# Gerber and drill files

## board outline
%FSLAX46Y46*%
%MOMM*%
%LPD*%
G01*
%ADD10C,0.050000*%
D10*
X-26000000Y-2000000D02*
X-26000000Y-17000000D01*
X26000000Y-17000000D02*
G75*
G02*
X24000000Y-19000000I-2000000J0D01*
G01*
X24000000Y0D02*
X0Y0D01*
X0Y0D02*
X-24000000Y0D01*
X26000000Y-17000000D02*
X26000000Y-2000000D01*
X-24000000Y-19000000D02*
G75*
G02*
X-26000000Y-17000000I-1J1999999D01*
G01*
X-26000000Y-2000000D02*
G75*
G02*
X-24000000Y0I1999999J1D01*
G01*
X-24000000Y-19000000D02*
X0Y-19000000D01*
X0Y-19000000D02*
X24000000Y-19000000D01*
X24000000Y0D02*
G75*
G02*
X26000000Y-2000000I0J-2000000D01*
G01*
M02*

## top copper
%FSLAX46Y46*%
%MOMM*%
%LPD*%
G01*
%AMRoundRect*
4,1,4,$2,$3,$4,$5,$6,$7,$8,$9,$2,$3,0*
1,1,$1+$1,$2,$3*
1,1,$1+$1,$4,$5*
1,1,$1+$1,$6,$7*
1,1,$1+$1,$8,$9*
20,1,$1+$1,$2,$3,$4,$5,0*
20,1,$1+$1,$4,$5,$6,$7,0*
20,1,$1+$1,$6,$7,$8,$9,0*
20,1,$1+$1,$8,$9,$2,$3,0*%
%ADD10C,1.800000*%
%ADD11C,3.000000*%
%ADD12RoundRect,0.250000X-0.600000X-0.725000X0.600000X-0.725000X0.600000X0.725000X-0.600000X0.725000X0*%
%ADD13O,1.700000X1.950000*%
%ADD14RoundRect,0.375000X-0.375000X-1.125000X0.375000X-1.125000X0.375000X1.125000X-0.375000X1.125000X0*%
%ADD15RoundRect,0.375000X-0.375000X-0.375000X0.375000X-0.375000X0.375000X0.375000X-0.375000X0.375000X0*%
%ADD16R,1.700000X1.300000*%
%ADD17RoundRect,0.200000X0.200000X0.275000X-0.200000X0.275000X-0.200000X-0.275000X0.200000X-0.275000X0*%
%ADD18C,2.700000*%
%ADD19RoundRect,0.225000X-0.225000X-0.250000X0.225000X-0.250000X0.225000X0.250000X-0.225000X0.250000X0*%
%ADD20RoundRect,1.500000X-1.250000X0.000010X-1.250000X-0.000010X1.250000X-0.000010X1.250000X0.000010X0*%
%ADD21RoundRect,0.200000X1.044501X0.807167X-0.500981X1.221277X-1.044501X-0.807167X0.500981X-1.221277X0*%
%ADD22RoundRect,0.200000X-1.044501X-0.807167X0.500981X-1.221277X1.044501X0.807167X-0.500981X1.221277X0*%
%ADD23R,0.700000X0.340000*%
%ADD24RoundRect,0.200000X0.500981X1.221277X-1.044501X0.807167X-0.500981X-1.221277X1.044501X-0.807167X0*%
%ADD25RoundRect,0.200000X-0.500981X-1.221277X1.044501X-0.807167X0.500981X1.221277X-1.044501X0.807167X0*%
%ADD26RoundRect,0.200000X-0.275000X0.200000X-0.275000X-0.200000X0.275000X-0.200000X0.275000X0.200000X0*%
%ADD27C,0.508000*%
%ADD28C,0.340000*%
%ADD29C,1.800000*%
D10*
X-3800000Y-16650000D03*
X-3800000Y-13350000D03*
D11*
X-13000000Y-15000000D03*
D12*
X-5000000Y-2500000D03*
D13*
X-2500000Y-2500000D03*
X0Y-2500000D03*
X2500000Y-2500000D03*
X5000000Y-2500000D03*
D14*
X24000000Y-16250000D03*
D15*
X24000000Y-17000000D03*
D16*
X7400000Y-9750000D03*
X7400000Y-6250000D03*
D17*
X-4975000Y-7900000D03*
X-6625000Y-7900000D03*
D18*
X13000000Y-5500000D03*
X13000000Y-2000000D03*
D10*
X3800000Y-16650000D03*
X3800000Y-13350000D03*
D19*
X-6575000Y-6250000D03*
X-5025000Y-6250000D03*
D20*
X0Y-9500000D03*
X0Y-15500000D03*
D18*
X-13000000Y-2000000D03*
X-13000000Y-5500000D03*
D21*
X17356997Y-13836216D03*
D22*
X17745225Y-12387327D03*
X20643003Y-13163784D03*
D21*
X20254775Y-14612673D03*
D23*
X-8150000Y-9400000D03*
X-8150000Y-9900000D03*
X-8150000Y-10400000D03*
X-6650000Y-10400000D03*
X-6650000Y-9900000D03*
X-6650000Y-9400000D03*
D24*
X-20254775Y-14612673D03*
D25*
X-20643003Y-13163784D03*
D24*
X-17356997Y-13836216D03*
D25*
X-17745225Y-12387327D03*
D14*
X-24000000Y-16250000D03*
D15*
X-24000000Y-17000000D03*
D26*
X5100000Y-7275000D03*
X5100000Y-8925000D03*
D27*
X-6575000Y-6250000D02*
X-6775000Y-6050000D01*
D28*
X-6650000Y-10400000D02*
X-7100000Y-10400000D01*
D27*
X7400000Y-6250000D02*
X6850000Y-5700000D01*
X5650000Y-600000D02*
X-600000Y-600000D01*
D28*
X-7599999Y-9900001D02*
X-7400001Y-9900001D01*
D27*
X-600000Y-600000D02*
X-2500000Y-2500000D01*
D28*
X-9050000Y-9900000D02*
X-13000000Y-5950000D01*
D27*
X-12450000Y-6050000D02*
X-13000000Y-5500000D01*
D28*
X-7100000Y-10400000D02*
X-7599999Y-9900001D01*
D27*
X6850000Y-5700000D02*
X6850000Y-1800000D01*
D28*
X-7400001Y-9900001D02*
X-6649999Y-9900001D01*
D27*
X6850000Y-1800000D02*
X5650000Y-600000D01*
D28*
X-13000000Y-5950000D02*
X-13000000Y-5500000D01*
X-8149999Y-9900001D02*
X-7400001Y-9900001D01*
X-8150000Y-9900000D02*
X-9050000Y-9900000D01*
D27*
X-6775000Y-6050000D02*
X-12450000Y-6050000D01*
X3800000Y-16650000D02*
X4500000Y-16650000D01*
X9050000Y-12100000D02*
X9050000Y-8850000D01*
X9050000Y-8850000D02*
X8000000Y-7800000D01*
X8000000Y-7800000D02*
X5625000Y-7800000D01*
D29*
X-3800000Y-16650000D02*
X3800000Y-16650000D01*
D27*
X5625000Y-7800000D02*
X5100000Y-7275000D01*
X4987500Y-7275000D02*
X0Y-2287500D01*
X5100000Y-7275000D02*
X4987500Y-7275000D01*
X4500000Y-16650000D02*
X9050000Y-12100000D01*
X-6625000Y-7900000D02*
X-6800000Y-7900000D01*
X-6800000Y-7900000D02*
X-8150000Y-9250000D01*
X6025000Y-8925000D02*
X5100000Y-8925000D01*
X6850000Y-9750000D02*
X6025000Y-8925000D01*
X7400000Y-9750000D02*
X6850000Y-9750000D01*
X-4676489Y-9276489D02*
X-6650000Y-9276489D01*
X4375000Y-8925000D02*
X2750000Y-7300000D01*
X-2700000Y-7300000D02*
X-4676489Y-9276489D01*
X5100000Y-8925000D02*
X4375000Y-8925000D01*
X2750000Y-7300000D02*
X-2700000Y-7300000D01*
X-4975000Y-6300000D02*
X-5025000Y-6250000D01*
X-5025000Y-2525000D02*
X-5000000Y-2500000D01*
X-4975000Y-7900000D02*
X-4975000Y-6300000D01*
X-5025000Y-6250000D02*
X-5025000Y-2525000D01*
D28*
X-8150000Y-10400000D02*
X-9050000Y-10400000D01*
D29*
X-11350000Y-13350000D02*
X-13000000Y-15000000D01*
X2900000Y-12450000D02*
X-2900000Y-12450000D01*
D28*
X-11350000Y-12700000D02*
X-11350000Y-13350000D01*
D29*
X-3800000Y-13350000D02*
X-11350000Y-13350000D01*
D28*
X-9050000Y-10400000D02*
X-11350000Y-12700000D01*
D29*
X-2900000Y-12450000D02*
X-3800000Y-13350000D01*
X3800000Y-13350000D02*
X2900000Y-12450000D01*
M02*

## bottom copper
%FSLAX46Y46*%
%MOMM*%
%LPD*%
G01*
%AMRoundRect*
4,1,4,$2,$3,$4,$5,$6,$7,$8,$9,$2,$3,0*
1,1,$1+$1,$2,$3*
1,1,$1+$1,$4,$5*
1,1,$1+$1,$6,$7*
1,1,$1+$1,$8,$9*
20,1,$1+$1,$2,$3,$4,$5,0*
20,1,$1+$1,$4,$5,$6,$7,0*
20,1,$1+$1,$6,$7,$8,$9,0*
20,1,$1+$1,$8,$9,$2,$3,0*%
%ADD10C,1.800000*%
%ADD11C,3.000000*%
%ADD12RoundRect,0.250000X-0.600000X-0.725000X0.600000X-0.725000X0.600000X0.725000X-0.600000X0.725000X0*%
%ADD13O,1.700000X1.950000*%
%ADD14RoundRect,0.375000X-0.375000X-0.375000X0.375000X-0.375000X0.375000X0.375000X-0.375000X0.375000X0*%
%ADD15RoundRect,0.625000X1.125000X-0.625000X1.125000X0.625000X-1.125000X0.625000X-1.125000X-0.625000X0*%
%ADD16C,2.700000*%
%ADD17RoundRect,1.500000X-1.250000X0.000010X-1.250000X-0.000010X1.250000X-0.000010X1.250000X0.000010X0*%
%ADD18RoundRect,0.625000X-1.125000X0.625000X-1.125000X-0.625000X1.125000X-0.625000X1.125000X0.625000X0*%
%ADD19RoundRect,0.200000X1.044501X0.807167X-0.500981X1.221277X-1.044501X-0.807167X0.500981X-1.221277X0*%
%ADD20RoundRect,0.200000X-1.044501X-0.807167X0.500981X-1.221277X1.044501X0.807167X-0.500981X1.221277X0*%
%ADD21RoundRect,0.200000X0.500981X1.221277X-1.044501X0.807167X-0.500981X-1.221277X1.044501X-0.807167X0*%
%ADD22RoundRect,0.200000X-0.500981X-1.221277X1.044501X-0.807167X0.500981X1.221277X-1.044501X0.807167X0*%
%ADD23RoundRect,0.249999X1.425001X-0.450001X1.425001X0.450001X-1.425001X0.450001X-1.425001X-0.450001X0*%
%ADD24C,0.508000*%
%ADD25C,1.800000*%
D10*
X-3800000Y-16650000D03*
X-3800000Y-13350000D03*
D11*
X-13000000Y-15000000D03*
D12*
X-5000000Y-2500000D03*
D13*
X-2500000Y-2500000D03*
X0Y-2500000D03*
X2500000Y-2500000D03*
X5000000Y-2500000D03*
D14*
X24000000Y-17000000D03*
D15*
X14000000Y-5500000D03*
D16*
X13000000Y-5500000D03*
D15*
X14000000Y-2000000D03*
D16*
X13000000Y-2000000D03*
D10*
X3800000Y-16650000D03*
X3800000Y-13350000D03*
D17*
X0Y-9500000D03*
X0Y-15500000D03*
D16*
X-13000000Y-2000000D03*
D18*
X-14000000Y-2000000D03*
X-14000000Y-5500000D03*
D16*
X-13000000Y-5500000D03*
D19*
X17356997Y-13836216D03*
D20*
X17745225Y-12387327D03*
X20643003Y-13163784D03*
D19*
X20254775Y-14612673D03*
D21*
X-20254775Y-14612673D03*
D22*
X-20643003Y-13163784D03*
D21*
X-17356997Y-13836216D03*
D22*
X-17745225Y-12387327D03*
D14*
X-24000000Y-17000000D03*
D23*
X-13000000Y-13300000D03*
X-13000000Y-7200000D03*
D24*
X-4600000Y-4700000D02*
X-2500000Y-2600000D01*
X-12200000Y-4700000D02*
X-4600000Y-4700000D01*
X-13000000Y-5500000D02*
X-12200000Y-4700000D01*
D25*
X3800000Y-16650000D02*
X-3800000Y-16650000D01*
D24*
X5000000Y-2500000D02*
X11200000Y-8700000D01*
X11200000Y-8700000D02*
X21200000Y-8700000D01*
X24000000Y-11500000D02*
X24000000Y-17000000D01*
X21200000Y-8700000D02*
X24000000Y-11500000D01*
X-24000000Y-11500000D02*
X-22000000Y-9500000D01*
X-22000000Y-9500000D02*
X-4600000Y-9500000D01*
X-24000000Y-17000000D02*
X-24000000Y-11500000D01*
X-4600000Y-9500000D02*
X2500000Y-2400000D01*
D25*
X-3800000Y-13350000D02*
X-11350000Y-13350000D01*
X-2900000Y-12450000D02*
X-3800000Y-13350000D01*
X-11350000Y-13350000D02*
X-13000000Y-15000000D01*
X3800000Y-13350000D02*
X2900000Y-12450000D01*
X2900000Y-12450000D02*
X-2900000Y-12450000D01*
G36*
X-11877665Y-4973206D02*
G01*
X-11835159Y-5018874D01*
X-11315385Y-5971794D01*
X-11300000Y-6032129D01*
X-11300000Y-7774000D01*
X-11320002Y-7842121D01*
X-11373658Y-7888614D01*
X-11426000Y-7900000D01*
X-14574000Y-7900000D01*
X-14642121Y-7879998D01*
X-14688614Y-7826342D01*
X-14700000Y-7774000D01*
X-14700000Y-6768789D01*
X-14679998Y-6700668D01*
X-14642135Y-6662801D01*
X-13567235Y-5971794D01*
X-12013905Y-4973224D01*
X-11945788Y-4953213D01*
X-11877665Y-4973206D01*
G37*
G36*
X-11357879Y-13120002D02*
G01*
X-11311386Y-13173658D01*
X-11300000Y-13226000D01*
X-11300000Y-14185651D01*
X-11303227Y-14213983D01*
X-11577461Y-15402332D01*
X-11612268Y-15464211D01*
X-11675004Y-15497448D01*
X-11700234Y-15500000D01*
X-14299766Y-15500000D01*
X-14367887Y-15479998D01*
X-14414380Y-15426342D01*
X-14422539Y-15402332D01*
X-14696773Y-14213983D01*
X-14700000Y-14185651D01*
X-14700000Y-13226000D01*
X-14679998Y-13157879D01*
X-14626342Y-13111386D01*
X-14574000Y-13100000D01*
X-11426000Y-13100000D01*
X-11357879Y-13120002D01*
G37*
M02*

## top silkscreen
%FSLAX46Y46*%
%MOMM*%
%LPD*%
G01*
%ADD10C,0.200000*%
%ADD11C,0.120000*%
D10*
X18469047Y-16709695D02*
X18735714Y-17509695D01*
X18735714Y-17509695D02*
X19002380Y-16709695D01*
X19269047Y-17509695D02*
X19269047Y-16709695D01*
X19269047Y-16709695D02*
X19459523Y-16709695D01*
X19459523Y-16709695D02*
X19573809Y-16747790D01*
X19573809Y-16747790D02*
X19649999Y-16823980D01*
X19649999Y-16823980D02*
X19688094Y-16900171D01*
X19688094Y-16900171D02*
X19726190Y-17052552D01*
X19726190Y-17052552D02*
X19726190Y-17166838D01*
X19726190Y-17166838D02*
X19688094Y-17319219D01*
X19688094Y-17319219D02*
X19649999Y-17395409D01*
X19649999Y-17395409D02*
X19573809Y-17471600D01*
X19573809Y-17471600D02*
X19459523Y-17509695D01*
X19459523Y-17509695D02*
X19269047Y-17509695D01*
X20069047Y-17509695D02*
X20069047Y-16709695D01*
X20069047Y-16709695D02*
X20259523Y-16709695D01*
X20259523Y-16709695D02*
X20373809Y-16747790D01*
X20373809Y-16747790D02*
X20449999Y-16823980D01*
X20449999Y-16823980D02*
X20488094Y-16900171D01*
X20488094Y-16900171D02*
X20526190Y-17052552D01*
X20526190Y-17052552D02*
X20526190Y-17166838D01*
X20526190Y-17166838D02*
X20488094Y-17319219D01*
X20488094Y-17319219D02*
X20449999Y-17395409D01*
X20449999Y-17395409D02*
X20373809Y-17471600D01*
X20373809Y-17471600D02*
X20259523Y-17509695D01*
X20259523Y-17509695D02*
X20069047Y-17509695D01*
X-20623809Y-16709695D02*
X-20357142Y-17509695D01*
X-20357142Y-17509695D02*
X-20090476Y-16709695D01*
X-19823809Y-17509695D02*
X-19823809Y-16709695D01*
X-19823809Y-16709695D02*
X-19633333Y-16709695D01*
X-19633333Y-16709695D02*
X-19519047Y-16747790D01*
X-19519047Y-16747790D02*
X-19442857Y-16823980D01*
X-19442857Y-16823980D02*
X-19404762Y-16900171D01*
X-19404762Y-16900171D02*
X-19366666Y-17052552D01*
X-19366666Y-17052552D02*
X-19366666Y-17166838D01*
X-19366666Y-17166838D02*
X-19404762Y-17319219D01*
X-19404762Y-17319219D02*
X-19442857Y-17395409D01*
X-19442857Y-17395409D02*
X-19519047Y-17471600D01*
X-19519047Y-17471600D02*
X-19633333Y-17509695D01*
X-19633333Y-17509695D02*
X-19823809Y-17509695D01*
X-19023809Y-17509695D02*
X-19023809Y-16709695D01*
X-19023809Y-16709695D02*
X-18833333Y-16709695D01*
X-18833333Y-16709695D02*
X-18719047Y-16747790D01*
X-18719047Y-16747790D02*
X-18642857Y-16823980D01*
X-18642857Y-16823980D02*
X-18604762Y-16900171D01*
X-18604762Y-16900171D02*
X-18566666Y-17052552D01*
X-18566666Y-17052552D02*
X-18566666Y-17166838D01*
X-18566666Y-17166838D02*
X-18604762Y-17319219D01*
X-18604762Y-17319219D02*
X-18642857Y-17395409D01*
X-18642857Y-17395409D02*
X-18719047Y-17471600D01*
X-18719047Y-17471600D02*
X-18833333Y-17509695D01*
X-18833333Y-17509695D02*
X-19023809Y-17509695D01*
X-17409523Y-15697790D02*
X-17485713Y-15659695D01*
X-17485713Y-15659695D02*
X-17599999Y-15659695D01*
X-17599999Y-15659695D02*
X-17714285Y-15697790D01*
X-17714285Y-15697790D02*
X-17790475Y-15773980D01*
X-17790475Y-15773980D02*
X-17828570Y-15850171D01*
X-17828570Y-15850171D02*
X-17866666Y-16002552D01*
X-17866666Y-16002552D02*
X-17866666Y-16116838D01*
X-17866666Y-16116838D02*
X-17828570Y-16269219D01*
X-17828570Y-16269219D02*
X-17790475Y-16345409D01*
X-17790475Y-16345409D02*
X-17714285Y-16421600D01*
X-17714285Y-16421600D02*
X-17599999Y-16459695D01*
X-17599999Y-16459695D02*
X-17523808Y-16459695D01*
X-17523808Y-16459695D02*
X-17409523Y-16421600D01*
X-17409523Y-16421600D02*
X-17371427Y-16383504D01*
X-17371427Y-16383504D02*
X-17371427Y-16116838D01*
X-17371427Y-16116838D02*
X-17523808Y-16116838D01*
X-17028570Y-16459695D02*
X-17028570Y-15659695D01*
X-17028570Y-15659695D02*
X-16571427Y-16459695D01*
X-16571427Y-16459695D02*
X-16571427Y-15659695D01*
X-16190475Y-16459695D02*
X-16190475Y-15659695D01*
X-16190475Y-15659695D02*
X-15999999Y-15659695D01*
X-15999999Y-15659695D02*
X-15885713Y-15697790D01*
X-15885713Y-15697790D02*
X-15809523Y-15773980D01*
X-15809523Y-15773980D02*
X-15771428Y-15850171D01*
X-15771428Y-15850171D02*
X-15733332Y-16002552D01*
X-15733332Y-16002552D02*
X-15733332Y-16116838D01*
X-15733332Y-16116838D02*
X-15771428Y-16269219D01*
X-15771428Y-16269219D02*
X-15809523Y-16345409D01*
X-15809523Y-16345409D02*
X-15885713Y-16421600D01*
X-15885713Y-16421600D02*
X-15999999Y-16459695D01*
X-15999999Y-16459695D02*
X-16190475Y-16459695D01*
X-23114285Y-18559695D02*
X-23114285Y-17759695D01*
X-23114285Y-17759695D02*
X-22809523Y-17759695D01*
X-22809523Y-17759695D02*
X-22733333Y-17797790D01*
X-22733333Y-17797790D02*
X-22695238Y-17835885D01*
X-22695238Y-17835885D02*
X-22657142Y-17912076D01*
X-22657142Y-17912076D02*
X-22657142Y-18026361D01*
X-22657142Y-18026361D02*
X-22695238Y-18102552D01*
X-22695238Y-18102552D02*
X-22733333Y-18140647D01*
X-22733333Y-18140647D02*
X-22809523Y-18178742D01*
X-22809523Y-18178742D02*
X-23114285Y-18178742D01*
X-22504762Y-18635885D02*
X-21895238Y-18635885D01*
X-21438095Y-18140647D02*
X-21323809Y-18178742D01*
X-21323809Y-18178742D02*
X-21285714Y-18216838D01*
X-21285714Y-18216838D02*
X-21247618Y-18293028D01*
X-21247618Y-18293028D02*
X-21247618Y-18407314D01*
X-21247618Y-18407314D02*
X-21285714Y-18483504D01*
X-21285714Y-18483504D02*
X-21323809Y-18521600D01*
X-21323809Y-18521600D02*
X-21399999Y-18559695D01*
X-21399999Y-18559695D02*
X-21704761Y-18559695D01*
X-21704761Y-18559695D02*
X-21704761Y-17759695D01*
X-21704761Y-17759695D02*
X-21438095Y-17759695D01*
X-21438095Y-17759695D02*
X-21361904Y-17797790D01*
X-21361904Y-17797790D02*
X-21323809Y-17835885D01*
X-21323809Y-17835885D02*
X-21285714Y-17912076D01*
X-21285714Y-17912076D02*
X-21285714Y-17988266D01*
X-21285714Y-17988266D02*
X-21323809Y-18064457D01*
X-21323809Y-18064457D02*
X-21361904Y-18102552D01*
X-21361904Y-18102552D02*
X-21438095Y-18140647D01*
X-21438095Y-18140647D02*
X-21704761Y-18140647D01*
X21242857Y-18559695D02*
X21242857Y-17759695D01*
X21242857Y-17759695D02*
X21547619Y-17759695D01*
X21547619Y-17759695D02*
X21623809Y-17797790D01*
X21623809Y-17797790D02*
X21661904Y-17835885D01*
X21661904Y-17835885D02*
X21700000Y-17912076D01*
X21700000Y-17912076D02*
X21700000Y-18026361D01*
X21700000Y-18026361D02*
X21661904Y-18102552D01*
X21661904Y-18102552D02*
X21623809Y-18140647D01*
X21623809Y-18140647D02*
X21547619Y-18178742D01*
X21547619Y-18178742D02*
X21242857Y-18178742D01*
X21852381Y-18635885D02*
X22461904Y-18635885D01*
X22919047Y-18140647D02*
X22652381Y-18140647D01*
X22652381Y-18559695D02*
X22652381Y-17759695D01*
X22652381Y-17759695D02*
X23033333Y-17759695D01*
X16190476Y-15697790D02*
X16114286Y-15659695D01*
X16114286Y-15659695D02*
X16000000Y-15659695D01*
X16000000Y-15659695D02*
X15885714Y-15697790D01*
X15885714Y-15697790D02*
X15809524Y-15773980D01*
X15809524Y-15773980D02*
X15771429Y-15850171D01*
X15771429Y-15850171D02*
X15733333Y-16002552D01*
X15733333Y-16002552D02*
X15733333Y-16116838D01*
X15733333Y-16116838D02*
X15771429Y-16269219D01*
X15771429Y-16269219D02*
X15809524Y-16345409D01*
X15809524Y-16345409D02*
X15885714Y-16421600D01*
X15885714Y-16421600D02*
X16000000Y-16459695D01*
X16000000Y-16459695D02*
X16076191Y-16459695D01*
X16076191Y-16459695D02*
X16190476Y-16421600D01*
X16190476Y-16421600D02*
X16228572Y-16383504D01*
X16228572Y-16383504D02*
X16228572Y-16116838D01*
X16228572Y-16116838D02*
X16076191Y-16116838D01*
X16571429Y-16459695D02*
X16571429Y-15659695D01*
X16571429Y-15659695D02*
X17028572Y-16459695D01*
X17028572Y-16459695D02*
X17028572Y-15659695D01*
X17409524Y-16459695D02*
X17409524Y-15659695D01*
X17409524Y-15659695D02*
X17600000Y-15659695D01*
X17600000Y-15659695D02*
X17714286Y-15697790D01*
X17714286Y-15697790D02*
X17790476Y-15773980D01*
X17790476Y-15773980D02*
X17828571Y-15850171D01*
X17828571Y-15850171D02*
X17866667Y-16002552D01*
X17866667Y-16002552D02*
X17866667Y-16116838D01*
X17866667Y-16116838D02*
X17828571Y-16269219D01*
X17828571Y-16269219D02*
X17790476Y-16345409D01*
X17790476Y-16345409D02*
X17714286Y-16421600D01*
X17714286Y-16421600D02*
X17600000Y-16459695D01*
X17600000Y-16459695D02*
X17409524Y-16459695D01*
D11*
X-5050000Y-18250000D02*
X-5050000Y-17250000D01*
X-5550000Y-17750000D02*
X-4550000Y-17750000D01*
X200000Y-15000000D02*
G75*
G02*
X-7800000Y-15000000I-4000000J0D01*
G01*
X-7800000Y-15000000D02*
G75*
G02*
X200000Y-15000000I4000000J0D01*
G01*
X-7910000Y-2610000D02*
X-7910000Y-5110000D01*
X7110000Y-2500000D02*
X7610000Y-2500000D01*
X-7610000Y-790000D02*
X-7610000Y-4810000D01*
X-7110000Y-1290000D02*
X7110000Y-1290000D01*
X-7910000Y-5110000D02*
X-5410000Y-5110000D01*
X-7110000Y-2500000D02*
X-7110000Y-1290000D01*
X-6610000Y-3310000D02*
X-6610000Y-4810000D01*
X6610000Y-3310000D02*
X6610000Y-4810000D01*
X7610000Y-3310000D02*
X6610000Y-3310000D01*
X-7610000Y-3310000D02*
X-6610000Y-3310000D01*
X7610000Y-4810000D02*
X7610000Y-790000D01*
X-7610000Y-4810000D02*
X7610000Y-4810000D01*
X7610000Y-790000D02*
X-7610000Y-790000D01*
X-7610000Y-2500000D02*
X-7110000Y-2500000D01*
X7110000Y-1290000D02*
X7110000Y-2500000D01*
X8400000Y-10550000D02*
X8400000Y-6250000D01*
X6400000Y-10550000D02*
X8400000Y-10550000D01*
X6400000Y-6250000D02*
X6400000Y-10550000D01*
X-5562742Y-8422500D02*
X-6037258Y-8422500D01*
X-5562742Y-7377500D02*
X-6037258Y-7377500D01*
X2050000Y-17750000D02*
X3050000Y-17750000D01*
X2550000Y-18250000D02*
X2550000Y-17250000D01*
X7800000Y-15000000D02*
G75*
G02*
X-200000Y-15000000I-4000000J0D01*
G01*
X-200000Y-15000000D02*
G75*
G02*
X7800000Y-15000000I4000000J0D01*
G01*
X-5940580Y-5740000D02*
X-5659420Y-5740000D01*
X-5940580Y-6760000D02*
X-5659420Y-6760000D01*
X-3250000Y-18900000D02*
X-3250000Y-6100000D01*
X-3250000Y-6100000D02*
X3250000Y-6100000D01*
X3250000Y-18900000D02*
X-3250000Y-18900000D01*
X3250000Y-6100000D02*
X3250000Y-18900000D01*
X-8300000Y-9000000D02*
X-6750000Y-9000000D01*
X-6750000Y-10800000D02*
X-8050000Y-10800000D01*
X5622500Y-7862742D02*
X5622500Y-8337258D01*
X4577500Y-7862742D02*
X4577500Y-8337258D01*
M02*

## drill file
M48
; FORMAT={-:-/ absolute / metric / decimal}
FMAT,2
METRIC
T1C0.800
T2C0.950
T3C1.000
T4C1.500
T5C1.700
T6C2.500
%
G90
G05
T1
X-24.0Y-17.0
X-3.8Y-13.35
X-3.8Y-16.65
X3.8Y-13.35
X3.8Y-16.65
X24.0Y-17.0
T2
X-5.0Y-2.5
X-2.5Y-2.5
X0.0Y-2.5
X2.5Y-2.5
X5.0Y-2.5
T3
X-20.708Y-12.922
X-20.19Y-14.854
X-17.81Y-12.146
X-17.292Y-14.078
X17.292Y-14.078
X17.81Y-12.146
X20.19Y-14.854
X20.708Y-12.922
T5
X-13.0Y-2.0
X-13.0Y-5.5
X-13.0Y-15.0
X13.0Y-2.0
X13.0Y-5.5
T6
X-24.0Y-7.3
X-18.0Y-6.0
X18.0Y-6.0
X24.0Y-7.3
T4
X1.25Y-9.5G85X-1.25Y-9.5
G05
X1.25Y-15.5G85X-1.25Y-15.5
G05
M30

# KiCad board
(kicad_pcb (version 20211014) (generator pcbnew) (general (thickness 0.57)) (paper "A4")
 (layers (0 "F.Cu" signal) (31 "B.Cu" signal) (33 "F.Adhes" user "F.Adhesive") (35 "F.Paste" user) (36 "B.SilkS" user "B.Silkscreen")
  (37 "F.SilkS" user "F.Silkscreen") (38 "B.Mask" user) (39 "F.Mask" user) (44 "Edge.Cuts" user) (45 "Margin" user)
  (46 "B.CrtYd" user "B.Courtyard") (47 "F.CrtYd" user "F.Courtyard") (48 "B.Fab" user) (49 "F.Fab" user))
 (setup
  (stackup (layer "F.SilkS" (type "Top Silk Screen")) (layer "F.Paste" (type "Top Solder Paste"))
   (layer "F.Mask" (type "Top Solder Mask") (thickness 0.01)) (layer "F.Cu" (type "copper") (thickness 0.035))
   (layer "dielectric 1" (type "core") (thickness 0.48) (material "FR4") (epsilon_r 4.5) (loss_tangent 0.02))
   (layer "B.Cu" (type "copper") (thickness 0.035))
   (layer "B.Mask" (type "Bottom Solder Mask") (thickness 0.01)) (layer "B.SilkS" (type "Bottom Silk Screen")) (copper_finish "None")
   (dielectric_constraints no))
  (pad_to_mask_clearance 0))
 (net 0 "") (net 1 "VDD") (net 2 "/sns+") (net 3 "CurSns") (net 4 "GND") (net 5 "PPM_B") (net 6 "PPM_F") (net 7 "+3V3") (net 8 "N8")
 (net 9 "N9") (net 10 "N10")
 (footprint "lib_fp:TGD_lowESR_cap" (layer "F.Cu") (at -3.8 15 90)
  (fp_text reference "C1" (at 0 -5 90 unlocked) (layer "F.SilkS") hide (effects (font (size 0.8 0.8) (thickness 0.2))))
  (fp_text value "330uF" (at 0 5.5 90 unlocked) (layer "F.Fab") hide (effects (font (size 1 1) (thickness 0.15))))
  (fp_line (start -3.25 -1.25) (end -2.25 -1.25) (layer "F.SilkS") (width 0.12))
  (fp_line (start -2.75 -1.75) (end -2.75 -0.75) (layer "F.SilkS") (width 0.12))
  (fp_circle (center 0 0) (end 4 0) (layer "F.SilkS") (width 0.12) (fill none))
  (pad "1" thru_hole circle (at -1.65 0 90) (size 1.8 1.8) (drill 0.8) (layers *.Cu *.Mask) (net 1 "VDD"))
  (pad "2" thru_hole circle (at 1.65 0 90) (size 1.8 1.8) (drill 0.8) (layers *.Cu *.Mask) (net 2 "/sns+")))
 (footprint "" (layer "F.Cu") (at -13 15)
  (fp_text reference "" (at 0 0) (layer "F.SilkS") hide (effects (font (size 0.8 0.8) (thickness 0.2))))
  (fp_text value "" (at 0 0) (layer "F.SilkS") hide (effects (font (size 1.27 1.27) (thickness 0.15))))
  (pad "2" thru_hole circle (at 0 0 270) (size 3 3) (drill 1.7) (layers *.Cu *.Mask) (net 2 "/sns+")))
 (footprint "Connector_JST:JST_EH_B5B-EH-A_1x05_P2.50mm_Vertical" (layer "F.Cu") (at -5 2.5)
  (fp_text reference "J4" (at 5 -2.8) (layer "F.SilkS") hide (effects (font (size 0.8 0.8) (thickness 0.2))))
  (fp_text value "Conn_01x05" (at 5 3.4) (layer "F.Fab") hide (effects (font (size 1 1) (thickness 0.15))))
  (fp_line (start -2.91 0.11) (end -2.91 2.61) (layer "F.SilkS") (width 0.12))
  (fp_line (start 12.11 0) (end 12.61 0) (layer "F.SilkS") (width 0.12))
  (fp_line (start -2.61 -1.71) (end -2.61 2.31) (layer "F.SilkS") (width 0.12))
  (fp_line (start -2.11 -1.21) (end 12.11 -1.21) (layer "F.SilkS") (width 0.12))
  (fp_line (start -2.91 2.61) (end -0.41 2.61) (layer "F.SilkS") (width 0.12))
  (fp_line (start -2.11 0) (end -2.11 -1.21) (layer "F.SilkS") (width 0.12))
  (fp_line (start -1.61 0.81) (end -1.61 2.31) (layer "F.SilkS") (width 0.12))
  (fp_line (start 11.61 0.81) (end 11.61 2.31) (layer "F.SilkS") (width 0.12))
  (fp_line (start 12.61 0.81) (end 11.61 0.81) (layer "F.SilkS") (width 0.12))
  (fp_line (start -2.61 0.81) (end -1.61 0.81) (layer "F.SilkS") (width 0.12))
  (fp_line (start 12.61 2.31) (end 12.61 -1.71) (layer "F.SilkS") (width 0.12))
  (fp_line (start -2.61 2.31) (end 12.61 2.31) (layer "F.SilkS") (width 0.12))
  (fp_line (start 12.61 -1.71) (end -2.61 -1.71) (layer "F.SilkS") (width 0.12))
  (fp_line (start -2.61 0) (end -2.11 0) (layer "F.SilkS") (width 0.12))
  (fp_line (start 12.11 -1.21) (end 12.11 0) (layer "F.SilkS") (width 0.12))
  (pad "1" thru_hole roundrect (at 0 0) (size 1.7 1.95) (drill 0.95) (layers *.Cu *.Mask) (roundrect_rratio 0.1470588235) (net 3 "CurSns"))
  (pad "2" thru_hole oval (at 2.5 0) (size 1.7 1.95) (drill 0.95) (layers *.Cu *.Mask) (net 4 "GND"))
  (pad "3" thru_hole oval (at 5 0) (size 1.7 1.95) (drill 0.95) (layers *.Cu *.Mask) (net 1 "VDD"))
  (pad "4" thru_hole oval (at 7.5 0) (size 1.7 1.95) (drill 0.95) (layers *.Cu *.Mask) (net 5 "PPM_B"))
  (pad "5" thru_hole oval (at 10 0) (size 1.7 1.95) (drill 0.95) (layers *.Cu *.Mask) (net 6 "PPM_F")))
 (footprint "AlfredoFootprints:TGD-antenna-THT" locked (layer "F.Cu") (at 24 16.25)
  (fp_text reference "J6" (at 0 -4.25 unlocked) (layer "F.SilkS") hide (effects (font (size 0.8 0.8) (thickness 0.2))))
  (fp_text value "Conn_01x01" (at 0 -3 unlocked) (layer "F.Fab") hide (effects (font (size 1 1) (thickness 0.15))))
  (pad "1" smd roundrect locked (at 0 0) (size 1.5 3) (layers "F.Cu" "F.Paste" "F.Mask") (roundrect_rratio 0.25) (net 6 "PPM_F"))
  (pad "1" thru_hole roundrect locked (at 0 0.75) (size 1.5 1.5) (drill 0.8) (layers *.Cu *.Mask) (roundrect_rratio 0.25) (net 6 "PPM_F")))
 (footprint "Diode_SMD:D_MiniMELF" (layer "F.Cu") (at 7.4 8 90)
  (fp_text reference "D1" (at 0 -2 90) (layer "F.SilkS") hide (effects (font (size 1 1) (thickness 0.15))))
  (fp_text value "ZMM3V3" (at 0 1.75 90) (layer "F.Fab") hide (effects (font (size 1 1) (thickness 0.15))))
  (fp_line (start -2.55 1) (end 1.75 1) (layer "F.SilkS") (width 0.12))
  (fp_line (start -2.55 -1) (end -2.55 1) (layer "F.SilkS") (width 0.12))
  (fp_line (start 1.75 -1) (end -2.55 -1) (layer "F.SilkS") (width 0.12))
  (pad "1" smd rect (at -1.75 0 90) (size 1.3 1.7) (layers "F.Cu" "F.Paste" "F.Mask") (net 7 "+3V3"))
  (pad "2" smd rect (at 1.75 0 90) (size 1.3 1.7) (layers "F.Cu" "F.Paste" "F.Mask") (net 4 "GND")))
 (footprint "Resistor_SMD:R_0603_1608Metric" (layer "F.Cu") (at -5.8 7.9 180)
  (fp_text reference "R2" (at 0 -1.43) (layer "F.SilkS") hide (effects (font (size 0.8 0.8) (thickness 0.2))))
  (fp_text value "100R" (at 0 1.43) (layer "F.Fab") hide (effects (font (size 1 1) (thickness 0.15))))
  (fp_line (start -0.237258 -0.5225) (end 0.237258 -0.5225) (layer "F.SilkS") (width 0.12))
  (fp_line (start -0.237258 0.5225) (end 0.237258 0.5225) (layer "F.SilkS") (width 0.12))
  (pad "1" smd roundrect (at -0.825 0 180) (size 0.8 0.95) (layers "F.Cu" "F.Paste" "F.Mask") (roundrect_rratio 0.25) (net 3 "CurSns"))
  (pad "2" smd roundrect (at 0.825 0 180) (size 0.8 0.95) (layers "F.Cu" "F.Paste" "F.Mask") (roundrect_rratio 0.25) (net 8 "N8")))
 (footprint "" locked (layer "F.Cu") (at 24 7.3)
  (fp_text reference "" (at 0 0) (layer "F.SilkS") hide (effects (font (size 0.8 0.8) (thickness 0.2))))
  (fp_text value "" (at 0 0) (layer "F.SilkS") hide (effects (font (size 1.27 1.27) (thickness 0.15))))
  (pad "" np_thru_hole circle locked (at 0 0 270) (size 2.2 2.2) (drill 2.5) (layers F&B.Cu *.Mask)))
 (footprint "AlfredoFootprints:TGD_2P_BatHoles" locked (layer "F.Cu") (at 13 3.75 90)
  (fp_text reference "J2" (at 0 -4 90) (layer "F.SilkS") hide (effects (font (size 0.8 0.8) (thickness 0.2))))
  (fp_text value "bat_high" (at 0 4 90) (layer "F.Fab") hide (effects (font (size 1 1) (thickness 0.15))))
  (pad "1" smd roundrect locked (at -1.75 1 90) (size 2.5 3.5) (layers "B.Cu" "B.Paste" "B.Mask") (roundrect_rratio 0.25) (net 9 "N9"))
  (pad "1" thru_hole circle locked (at -1.75 0 90) (size 2.7 2.7) (drill 1.7) (layers *.Cu *.Mask) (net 9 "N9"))
  (pad "2" smd roundrect locked (at 1.75 1 90) (size 2.5 3.5) (layers "B.Cu" "B.Paste" "B.Mask") (roundrect_rratio 0.25) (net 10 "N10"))
  (pad "2" thru_hole circle locked (at 1.75 0 90) (size 2.7 2.7) (drill 1.7) (layers *.Cu *.Mask) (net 10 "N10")))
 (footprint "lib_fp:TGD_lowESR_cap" (layer "F.Cu") (at 3.8 15 90)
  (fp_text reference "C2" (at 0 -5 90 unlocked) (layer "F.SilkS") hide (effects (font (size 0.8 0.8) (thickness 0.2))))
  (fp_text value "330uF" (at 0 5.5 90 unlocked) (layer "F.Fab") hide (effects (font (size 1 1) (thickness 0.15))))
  (fp_line (start -2.75 -1.75) (end -2.75 -0.75) (layer "F.SilkS") (width 0.12))
  (fp_line (start -3.25 -1.25) (end -2.25 -1.25) (layer "F.SilkS") (width 0.12))
  (fp_circle (center 0 0) (end 4 0) (layer "F.SilkS") (width 0.12) (fill none))
  (pad "1" thru_hole circle (at -1.65 0 90) (size 1.8 1.8) (drill 0.8) (layers *.Cu *.Mask) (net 1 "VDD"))
  (pad "2" thru_hole circle (at 1.65 0 90) (size 1.8 1.8) (drill 0.8) (layers *.Cu *.Mask) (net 2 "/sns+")))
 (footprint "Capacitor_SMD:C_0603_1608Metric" (layer "F.Cu") (at -5.8 6.25)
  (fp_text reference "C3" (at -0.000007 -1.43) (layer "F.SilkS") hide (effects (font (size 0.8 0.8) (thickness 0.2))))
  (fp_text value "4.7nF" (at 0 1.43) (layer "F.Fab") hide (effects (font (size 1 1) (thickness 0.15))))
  (fp_line (start -0.14058 -0.51) (end 0.14058 -0.51) (layer "F.SilkS") (width 0.12))
  (fp_line (start -0.14058 0.51) (end 0.14058 0.51) (layer "F.SilkS") (width 0.12))
  (pad "1" smd roundrect (at -0.775 0) (size 0.9 0.95) (layers "F.Cu" "F.Paste" "F.Mask") (roundrect_rratio 0.25) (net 4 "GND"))
  (pad "2" smd roundrect (at 0.775 0) (size 0.9 0.95) (layers "F.Cu" "F.Paste" "F.Mask") (roundrect_rratio 0.25) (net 3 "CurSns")))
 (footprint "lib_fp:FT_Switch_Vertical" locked (layer "F.Cu") (at 0 9.5 -90)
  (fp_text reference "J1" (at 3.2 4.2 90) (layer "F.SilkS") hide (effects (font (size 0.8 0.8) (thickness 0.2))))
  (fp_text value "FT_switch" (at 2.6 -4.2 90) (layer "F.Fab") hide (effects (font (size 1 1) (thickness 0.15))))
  (fp_line (start 9.4 3.25) (end -3.4 3.25) (layer "F.SilkS") (width 0.12))
  (fp_line (start -3.4 3.25) (end -3.4 -3.25) (layer "F.SilkS") (width 0.12))
  (fp_line (start 9.4 -3.25) (end 9.4 3.25) (layer "F.SilkS") (width 0.12))
  (fp_line (start -3.4 -3.25) (end 9.4 -3.25) (layer "F.SilkS") (width 0.12))
  (pad "1" thru_hole roundrect locked (at 0 0 270) (size 3 5.5) (drill oval 1.5 4) (layers *.Cu *.Mask) (roundrect_rratio 0.5) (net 9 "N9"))
  (pad "2" thru_hole roundrect locked (at 6 0 270) (size 3 5.5) (drill oval 1.5 4) (layers *.Cu *.Mask) (roundrect_rratio 0.5) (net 1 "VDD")))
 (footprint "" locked (layer "F.Cu") (at -18 6)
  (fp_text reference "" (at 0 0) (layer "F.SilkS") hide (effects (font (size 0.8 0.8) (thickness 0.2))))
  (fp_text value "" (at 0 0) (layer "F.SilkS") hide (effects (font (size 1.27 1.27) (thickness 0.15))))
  (pad "" np_thru_hole circle locked (at 0 0 270) (size 2.5 2.5) (drill 2.5) (layers F&B.Cu *.Mask)))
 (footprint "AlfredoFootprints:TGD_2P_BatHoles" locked (layer "F.Cu") (at -13 3.75 -90)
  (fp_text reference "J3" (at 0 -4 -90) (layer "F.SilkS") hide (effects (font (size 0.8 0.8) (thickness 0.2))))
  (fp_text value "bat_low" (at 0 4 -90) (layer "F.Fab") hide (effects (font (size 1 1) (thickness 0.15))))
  (pad "1" thru_hole circle locked (at -1.75 0 270) (size 2.7 2.7) (drill 1.7) (layers *.Cu *.Mask) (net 10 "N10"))
  (pad "1" smd roundrect locked (at -1.75 1 270) (size 2.5 3.5) (layers "B.Cu" "B.Paste" "B.Mask") (roundrect_rratio 0.25) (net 10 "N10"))
  (pad "2" smd roundrect locked (at 1.75 1 270) (size 2.5 3.5) (layers "B.Cu" "B.Paste" "B.Mask") (roundrect_rratio 0.25) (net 4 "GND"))
  (pad "2" thru_hole circle locked (at 1.75 0 270) (size 2.7 2.7) (drill 1.7) (layers *.Cu *.Mask) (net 4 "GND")))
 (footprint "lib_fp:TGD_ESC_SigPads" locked (layer "F.Cu") (at 19 13.5 -15)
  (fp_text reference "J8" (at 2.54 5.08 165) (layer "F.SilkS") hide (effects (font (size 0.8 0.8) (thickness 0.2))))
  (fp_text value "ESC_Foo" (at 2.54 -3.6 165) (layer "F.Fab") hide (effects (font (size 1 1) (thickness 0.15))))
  (pad "1" thru_hole roundrect locked (at -1.5 1 165) (size 2 2.5) (drill 1 (offset 0 0.25)) (layers *.Cu *.Mask) (roundrect_rratio 0.1)
   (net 2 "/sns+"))
  (pad "1" thru_hole roundrect locked (at -1.5 -1 345) (size 2 2.5) (drill 1 (offset 0 0.25)) (layers *.Cu *.Mask) (roundrect_rratio 0.1)
   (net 2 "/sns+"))
  (pad "2" thru_hole roundrect locked (at 1.5 -1 345) (size 2 2.5) (drill 1 (offset 0 0.25)) (layers *.Cu *.Mask) (roundrect_rratio 0.1)
   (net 1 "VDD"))
  (pad "2" thru_hole roundrect locked (at 1.5 1 165) (size 2 2.5) (drill 1 (offset 0 0.25)) (layers *.Cu *.Mask) (roundrect_rratio 0.1)
   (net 1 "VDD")))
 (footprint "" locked (layer "F.Cu") (at 17.5 6)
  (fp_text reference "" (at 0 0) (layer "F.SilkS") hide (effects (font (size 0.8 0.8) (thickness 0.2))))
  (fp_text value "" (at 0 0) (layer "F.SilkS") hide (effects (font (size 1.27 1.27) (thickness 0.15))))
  (pad "" np_thru_hole circle locked (at 0.5 0 270) (size 2.2 2.2) (drill 2.5) (layers F&B.Cu *.Mask)))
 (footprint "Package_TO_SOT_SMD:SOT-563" (layer "F.Cu") (at -7.4 9.9)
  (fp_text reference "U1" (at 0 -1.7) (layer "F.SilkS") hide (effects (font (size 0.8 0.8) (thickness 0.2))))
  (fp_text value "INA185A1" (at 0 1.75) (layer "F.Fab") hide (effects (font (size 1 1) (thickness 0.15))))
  (fp_line (start -0.9 -0.9) (end 0.65 -0.9) (layer "F.SilkS") (width 0.12))
  (fp_line (start 0.65 0.9) (end -0.65 0.9) (layer "F.SilkS") (width 0.12))
  (pad "1" smd rect (at -0.75 -0.5) (size 0.7 0.34) (layers "F.Cu" "F.Paste" "F.Mask") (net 8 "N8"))
  (pad "2" smd rect (at -0.75 0) (size 0.7 0.34) (layers "F.Cu" "F.Paste" "F.Mask") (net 4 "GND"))
  (pad "3" smd rect (at -0.75 0.5) (size 0.7 0.34) (layers "F.Cu" "F.Paste" "F.Mask") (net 2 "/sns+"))
  (pad "4" smd rect (at 0.75 0.5) (size 0.7 0.34) (layers "F.Cu" "F.Paste" "F.Mask") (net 4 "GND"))
  (pad "5" smd rect (at 0.75 0) (size 0.7 0.34) (layers "F.Cu" "F.Paste" "F.Mask") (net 4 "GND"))
  (pad "6" smd rect (at 0.75 -0.5) (size 0.7 0.34) (layers "F.Cu" "F.Paste" "F.Mask") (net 7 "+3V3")))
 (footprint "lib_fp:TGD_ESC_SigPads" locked (layer "F.Cu") (at -19 13.5 15)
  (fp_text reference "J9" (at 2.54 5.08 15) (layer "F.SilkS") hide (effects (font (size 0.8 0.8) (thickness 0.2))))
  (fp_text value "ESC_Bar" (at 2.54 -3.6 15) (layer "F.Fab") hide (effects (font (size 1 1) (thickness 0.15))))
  (pad "1" thru_hole roundrect locked (at -1.5 1 195) (size 2 2.5) (drill 1 (offset 0 0.25)) (layers *.Cu *.Mask) (roundrect_rratio 0.1)
   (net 1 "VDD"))
  (pad "1" thru_hole roundrect locked (at -1.5 -1 15) (size 2 2.5) (drill 1 (offset 0 0.25)) (layers *.Cu *.Mask) (roundrect_rratio 0.1)
   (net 1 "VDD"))
  (pad "2" thru_hole roundrect locked (at 1.5 1 195) (size 2 2.5) (drill 1 (offset 0 0.25)) (layers *.Cu *.Mask) (roundrect_rratio 0.1)
   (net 2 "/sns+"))
  (pad "2" thru_hole roundrect locked (at 1.5 -1 15) (size 2 2.5) (drill 1 (offset 0 0.25)) (layers *.Cu *.Mask) (roundrect_rratio 0.1)
   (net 2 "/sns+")))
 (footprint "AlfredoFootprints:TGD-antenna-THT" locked (layer "F.Cu") (at -24 16.25)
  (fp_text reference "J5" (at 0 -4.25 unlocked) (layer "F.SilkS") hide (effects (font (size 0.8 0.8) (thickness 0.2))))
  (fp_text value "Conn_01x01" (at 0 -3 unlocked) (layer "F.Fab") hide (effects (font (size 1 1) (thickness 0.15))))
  (pad "1" smd roundrect locked (at 0 0) (size 1.5 3) (layers "F.Cu" "F.Paste" "F.Mask") (roundrect_rratio 0.25) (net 5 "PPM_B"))
  (pad "1" thru_hole roundrect locked (at 0 0.75) (size 1.5 1.5) (drill 0.8) (layers *.Cu *.Mask) (roundrect_rratio 0.25) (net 5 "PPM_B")))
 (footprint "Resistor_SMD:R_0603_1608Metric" (layer "F.Cu") (at 5.1 8.1 -90)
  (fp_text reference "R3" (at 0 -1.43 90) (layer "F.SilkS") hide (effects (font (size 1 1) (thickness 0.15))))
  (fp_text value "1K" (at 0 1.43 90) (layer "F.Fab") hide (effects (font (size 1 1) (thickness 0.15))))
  (fp_line (start -0.237258 -0.5225) (end 0.237258 -0.5225) (layer "F.SilkS") (width 0.12))
  (fp_line (start -0.237258 0.5225) (end 0.237258 0.5225) (layer "F.SilkS") (width 0.12))
  (pad "1" smd roundrect (at -0.825 0 270) (size 0.8 0.95) (layers "F.Cu" "F.Paste" "F.Mask") (roundrect_rratio 0.25) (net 1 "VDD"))
  (pad "2" smd roundrect (at 0.825 0 270) (size 0.8 0.95) (layers "F.Cu" "F.Paste" "F.Mask") (roundrect_rratio 0.25) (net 7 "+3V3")))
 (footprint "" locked (layer "F.Cu") (at -24.5 7.3)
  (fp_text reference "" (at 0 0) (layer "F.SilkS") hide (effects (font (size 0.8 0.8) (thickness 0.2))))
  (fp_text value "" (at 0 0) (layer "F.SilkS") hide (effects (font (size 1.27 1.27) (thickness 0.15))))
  (pad "" np_thru_hole circle locked (at 0.5 0 270) (size 2.2 2.2) (drill 2.5) (layers F&B.Cu *.Mask)))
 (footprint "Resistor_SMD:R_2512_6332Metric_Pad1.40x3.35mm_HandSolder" (layer "B.Cu") (at -13 10.25 90)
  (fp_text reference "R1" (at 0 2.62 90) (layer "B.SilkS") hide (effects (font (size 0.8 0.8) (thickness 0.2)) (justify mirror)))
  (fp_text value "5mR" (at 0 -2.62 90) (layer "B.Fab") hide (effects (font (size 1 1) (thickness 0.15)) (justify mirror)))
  (pad "1" smd roundrect (at -3.05 0 90) (size 1.4 3.35) (layers "B.Cu" "B.Paste" "B.Mask") (roundrect_rratio 0.1785707143) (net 2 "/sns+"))
  (pad "2" smd roundrect (at 3.05 0 90) (size 1.4 3.35) (layers "B.Cu" "B.Paste" "B.Mask") (roundrect_rratio 0.1785707143) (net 4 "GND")))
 (gr_line (start -26 2) (end -26 17) (layer "Edge.Cuts") (width 0.05))
 (gr_arc (start 26 17) (mid 25.414214 18.414214) (end 24 19) (layer "Edge.Cuts") (width 0.05))
 (gr_line (start 24 0) (end 0 0) (layer "Edge.Cuts") (width 0.05))
 (gr_line (start 0 0) (end -24 0) (layer "Edge.Cuts") (width 0.05))
 (gr_line (start 26 17) (end 26 2) (layer "Edge.Cuts") (width 0.05))
 (gr_arc (start -24 19) (mid -25.414214 18.414214) (end -26 17) (layer "Edge.Cuts") (width 0.05))
 (gr_arc (start -26 2) (mid -25.414214 0.585786) (end -24 0) (layer "Edge.Cuts") (width 0.05))
 (gr_line (start -24 19) (end 0 19) (layer "Edge.Cuts") (width 0.05))
 (gr_line (start 0 19) (end 24 19) (layer "Edge.Cuts") (width 0.05))
 (gr_arc (start 24 0) (mid 25.414214 0.585786) (end 26 2) (layer "Edge.Cuts") (width 0.05))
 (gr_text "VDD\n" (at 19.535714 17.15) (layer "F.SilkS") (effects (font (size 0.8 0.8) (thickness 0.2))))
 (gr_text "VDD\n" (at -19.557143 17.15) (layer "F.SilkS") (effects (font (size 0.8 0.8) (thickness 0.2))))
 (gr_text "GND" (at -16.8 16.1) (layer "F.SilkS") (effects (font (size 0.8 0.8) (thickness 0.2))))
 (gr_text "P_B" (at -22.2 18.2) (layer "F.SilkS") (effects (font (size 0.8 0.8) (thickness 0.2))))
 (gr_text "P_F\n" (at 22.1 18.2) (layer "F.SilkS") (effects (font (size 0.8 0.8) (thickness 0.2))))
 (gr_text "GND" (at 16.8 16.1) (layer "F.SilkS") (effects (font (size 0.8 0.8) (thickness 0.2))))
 (segment (start -6.575 6.25) (end -6.775 6.05) (width 0.508) (layer "F.Cu") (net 4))
 (segment (start -6.65 10.4) (end -7.1 10.4) (width 0.34) (layer "F.Cu") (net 4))
 (segment (start 7.4 6.25) (end 6.85 5.7) (width 0.508) (layer "F.Cu") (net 4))
 (segment (start 5.65 0.6) (end -0.6 0.6) (width 0.508) (layer "F.Cu") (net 4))
 (segment (start -7.599999 9.900001) (end -7.400001 9.900001) (width 0.34) (layer "F.Cu") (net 4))
 (segment (start -0.6 0.6) (end -2.5 2.5) (width 0.508) (layer "F.Cu") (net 4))
 (segment (start -9.05 9.9) (end -13 5.95) (width 0.34) (layer "F.Cu") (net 4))
 (segment (start -12.45 6.05) (end -13 5.5) (width 0.508) (layer "F.Cu") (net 4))
 (segment (start -7.1 10.4) (end -7.599999 9.900001) (width 0.34) (layer "F.Cu") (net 4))
 (segment (start 6.85 5.7) (end 6.85 1.8) (width 0.508) (layer "F.Cu") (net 4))
 (segment (start -7.400001 9.900001) (end -6.649999 9.900001) (width 0.34) (layer "F.Cu") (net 4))
 (segment (start 6.85 1.8) (end 5.65 0.6) (width 0.508) (layer "F.Cu") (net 4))
 (segment (start -13 5.95) (end -13 5.5) (width 0.34) (layer "F.Cu") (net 4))
 (segment (start -8.149999 9.900001) (end -7.400001 9.900001) (width 0.34) (layer "F.Cu") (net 4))
 (segment (start -8.15 9.9) (end -9.05 9.9) (width 0.34) (layer "F.Cu") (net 4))
 (segment (start -6.775 6.05) (end -12.45 6.05) (width 0.508) (layer "F.Cu") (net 4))
 (segment (start -4.6 4.7) (end -2.5 2.6) (width 0.508) (layer "B.Cu") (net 4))
 (segment (start -12.2 4.7) (end -4.6 4.7) (width 0.508) (layer "B.Cu") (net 4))
 (segment (start -13 5.5) (end -12.2 4.7) (width 0.508) (layer "B.Cu") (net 4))
 (segment (start 3.8 16.65) (end 4.5 16.65) (width 0.508) (layer "F.Cu") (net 1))
 (segment (start 9.05 12.1) (end 9.05 8.85) (width 0.508) (layer "F.Cu") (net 1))
 (segment (start 9.05 8.85) (end 8 7.8) (width 0.508) (layer "F.Cu") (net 1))
 (segment (start 8 7.8) (end 5.625 7.8) (width 0.508) (layer "F.Cu") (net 1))
 (segment (start -3.8 16.65) (end 3.8 16.65) (width 1.8) (layer "F.Cu") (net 1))
 (segment (start 5.625 7.8) (end 5.1 7.275) (width 0.508) (layer "F.Cu") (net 1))
 (segment (start 4.9875 7.275) (end 0 2.2875) (width 0.508) (layer "F.Cu") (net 1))
 (segment (start 5.1 7.275) (end 4.9875 7.275) (width 0.508) (layer "F.Cu") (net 1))
 (segment (start 4.5 16.65) (end 9.05 12.1) (width 0.508) (layer "F.Cu") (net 1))
 (segment (start 3.8 16.65) (end -3.8 16.65) (width 1.8) (layer "B.Cu") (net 1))
 (segment (start 5 2.5) (end 11.2 8.7) (width 0.508) (layer "B.Cu") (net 6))
 (segment (start 11.2 8.7) (end 21.2 8.7) (width 0.508) (layer "B.Cu") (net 6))
 (segment (start 24 11.5) (end 24 17) (width 0.508) (layer "B.Cu") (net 6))
 (segment (start 21.2 8.7) (end 24 11.5) (width 0.508) (layer "B.Cu") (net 6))
 (segment (start -24 11.5) (end -22 9.5) (width 0.508) (layer "B.Cu") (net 5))
 (segment (start -22 9.5) (end -4.6 9.5) (width 0.508) (layer "B.Cu") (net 5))
 (segment (start -24 17) (end -24 11.5) (width 0.508) (layer "B.Cu") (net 5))
 (segment (start -4.6 9.5) (end 2.5 2.4) (width 0.508) (layer "B.Cu") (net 5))
 (segment (start -6.625 7.9) (end -6.8 7.9) (width 0.508) (layer "F.Cu") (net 8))
 (segment (start -6.8 7.9) (end -8.15 9.25) (width 0.508) (layer "F.Cu") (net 8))
 (segment (start 6.025 8.925) (end 5.1 8.925) (width 0.508) (layer "F.Cu") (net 7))
 (segment (start 6.85 9.75) (end 6.025 8.925) (width 0.508) (layer "F.Cu") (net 7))
 (segment (start 7.4 9.75) (end 6.85 9.75) (width 0.508) (layer "F.Cu") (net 7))
 (segment (start -4.676489 9.276489) (end -6.65 9.276489) (width 0.508) (layer "F.Cu") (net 7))
 (segment (start 4.375 8.925) (end 2.75 7.3) (width 0.508) (layer "F.Cu") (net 7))
 (segment (start -2.7 7.3) (end -4.676489 9.276489) (width 0.508) (layer "F.Cu") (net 7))
 (segment (start 5.1 8.925) (end 4.375 8.925) (width 0.508) (layer "F.Cu") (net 7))
 (segment (start 2.75 7.3) (end -2.7 7.3) (width 0.508) (layer "F.Cu") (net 7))
 (segment (start -4.975 6.3) (end -5.025 6.25) (width 0.508) (layer "F.Cu") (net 3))
 (segment (start -5.025 2.525) (end -5 2.5) (width 0.508) (layer "F.Cu") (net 3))
 (segment (start -4.975 7.9) (end -4.975 6.3) (width 0.508) (layer "F.Cu") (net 3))
 (segment (start -5.025 6.25) (end -5.025 2.525) (width 0.508) (layer "F.Cu") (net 3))
 (segment (start -8.15 10.4) (end -9.05 10.4) (width 0.34) (layer "F.Cu") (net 2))
 (segment (start -11.35 13.35) (end -13 15) (width 1.8) (layer "F.Cu") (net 2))
 (segment (start 2.9 12.45) (end -2.9 12.45) (width 1.8) (layer "F.Cu") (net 2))
 (segment (start -11.35 12.7) (end -11.35 13.35) (width 0.34) (layer "F.Cu") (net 2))
 (segment (start -3.8 13.35) (end -11.35 13.35) (width 1.8) (layer "F.Cu") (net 2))
 (segment (start -9.05 10.4) (end -11.35 12.7) (width 0.34) (layer "F.Cu") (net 2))
 (segment (start -2.9 12.45) (end -3.8 13.35) (width 1.8) (layer "F.Cu") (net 2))
 (segment (start 3.8 13.35) (end 2.9 12.45) (width 1.8) (layer "F.Cu") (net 2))
 (segment (start -3.8 13.35) (end -11.35 13.35) (width 1.8) (layer "B.Cu") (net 2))
 (segment (start -2.9 12.45) (end -3.8 13.35) (width 1.8) (layer "B.Cu") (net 2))
 (segment (start -11.35 13.35) (end -13 15) (width 1.8) (layer "B.Cu") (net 2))
 (segment (start 3.8 13.35) (end 2.9 12.45) (width 1.8) (layer "B.Cu") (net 2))
 (segment (start 2.9 12.45) (end -2.9 12.45) (width 1.8) (layer "B.Cu") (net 2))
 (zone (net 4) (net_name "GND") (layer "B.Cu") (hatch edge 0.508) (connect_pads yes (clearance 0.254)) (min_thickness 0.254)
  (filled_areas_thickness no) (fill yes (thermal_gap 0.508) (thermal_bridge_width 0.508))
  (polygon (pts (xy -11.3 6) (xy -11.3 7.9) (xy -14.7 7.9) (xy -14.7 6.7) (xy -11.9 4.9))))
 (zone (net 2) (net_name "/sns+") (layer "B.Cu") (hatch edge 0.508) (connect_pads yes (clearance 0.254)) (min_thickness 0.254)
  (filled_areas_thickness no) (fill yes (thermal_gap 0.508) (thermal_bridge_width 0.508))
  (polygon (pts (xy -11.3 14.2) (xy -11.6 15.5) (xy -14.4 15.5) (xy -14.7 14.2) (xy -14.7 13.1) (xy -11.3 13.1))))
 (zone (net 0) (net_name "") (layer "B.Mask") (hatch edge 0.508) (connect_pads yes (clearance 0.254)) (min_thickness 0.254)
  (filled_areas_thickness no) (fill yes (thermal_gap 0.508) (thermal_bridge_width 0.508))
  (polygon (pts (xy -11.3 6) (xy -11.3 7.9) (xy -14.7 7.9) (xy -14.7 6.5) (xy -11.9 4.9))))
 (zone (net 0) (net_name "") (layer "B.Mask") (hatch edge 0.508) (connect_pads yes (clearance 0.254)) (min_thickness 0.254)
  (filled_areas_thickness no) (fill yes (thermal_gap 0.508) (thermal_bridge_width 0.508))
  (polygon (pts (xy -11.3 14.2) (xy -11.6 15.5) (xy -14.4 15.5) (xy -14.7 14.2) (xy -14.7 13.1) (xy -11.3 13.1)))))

